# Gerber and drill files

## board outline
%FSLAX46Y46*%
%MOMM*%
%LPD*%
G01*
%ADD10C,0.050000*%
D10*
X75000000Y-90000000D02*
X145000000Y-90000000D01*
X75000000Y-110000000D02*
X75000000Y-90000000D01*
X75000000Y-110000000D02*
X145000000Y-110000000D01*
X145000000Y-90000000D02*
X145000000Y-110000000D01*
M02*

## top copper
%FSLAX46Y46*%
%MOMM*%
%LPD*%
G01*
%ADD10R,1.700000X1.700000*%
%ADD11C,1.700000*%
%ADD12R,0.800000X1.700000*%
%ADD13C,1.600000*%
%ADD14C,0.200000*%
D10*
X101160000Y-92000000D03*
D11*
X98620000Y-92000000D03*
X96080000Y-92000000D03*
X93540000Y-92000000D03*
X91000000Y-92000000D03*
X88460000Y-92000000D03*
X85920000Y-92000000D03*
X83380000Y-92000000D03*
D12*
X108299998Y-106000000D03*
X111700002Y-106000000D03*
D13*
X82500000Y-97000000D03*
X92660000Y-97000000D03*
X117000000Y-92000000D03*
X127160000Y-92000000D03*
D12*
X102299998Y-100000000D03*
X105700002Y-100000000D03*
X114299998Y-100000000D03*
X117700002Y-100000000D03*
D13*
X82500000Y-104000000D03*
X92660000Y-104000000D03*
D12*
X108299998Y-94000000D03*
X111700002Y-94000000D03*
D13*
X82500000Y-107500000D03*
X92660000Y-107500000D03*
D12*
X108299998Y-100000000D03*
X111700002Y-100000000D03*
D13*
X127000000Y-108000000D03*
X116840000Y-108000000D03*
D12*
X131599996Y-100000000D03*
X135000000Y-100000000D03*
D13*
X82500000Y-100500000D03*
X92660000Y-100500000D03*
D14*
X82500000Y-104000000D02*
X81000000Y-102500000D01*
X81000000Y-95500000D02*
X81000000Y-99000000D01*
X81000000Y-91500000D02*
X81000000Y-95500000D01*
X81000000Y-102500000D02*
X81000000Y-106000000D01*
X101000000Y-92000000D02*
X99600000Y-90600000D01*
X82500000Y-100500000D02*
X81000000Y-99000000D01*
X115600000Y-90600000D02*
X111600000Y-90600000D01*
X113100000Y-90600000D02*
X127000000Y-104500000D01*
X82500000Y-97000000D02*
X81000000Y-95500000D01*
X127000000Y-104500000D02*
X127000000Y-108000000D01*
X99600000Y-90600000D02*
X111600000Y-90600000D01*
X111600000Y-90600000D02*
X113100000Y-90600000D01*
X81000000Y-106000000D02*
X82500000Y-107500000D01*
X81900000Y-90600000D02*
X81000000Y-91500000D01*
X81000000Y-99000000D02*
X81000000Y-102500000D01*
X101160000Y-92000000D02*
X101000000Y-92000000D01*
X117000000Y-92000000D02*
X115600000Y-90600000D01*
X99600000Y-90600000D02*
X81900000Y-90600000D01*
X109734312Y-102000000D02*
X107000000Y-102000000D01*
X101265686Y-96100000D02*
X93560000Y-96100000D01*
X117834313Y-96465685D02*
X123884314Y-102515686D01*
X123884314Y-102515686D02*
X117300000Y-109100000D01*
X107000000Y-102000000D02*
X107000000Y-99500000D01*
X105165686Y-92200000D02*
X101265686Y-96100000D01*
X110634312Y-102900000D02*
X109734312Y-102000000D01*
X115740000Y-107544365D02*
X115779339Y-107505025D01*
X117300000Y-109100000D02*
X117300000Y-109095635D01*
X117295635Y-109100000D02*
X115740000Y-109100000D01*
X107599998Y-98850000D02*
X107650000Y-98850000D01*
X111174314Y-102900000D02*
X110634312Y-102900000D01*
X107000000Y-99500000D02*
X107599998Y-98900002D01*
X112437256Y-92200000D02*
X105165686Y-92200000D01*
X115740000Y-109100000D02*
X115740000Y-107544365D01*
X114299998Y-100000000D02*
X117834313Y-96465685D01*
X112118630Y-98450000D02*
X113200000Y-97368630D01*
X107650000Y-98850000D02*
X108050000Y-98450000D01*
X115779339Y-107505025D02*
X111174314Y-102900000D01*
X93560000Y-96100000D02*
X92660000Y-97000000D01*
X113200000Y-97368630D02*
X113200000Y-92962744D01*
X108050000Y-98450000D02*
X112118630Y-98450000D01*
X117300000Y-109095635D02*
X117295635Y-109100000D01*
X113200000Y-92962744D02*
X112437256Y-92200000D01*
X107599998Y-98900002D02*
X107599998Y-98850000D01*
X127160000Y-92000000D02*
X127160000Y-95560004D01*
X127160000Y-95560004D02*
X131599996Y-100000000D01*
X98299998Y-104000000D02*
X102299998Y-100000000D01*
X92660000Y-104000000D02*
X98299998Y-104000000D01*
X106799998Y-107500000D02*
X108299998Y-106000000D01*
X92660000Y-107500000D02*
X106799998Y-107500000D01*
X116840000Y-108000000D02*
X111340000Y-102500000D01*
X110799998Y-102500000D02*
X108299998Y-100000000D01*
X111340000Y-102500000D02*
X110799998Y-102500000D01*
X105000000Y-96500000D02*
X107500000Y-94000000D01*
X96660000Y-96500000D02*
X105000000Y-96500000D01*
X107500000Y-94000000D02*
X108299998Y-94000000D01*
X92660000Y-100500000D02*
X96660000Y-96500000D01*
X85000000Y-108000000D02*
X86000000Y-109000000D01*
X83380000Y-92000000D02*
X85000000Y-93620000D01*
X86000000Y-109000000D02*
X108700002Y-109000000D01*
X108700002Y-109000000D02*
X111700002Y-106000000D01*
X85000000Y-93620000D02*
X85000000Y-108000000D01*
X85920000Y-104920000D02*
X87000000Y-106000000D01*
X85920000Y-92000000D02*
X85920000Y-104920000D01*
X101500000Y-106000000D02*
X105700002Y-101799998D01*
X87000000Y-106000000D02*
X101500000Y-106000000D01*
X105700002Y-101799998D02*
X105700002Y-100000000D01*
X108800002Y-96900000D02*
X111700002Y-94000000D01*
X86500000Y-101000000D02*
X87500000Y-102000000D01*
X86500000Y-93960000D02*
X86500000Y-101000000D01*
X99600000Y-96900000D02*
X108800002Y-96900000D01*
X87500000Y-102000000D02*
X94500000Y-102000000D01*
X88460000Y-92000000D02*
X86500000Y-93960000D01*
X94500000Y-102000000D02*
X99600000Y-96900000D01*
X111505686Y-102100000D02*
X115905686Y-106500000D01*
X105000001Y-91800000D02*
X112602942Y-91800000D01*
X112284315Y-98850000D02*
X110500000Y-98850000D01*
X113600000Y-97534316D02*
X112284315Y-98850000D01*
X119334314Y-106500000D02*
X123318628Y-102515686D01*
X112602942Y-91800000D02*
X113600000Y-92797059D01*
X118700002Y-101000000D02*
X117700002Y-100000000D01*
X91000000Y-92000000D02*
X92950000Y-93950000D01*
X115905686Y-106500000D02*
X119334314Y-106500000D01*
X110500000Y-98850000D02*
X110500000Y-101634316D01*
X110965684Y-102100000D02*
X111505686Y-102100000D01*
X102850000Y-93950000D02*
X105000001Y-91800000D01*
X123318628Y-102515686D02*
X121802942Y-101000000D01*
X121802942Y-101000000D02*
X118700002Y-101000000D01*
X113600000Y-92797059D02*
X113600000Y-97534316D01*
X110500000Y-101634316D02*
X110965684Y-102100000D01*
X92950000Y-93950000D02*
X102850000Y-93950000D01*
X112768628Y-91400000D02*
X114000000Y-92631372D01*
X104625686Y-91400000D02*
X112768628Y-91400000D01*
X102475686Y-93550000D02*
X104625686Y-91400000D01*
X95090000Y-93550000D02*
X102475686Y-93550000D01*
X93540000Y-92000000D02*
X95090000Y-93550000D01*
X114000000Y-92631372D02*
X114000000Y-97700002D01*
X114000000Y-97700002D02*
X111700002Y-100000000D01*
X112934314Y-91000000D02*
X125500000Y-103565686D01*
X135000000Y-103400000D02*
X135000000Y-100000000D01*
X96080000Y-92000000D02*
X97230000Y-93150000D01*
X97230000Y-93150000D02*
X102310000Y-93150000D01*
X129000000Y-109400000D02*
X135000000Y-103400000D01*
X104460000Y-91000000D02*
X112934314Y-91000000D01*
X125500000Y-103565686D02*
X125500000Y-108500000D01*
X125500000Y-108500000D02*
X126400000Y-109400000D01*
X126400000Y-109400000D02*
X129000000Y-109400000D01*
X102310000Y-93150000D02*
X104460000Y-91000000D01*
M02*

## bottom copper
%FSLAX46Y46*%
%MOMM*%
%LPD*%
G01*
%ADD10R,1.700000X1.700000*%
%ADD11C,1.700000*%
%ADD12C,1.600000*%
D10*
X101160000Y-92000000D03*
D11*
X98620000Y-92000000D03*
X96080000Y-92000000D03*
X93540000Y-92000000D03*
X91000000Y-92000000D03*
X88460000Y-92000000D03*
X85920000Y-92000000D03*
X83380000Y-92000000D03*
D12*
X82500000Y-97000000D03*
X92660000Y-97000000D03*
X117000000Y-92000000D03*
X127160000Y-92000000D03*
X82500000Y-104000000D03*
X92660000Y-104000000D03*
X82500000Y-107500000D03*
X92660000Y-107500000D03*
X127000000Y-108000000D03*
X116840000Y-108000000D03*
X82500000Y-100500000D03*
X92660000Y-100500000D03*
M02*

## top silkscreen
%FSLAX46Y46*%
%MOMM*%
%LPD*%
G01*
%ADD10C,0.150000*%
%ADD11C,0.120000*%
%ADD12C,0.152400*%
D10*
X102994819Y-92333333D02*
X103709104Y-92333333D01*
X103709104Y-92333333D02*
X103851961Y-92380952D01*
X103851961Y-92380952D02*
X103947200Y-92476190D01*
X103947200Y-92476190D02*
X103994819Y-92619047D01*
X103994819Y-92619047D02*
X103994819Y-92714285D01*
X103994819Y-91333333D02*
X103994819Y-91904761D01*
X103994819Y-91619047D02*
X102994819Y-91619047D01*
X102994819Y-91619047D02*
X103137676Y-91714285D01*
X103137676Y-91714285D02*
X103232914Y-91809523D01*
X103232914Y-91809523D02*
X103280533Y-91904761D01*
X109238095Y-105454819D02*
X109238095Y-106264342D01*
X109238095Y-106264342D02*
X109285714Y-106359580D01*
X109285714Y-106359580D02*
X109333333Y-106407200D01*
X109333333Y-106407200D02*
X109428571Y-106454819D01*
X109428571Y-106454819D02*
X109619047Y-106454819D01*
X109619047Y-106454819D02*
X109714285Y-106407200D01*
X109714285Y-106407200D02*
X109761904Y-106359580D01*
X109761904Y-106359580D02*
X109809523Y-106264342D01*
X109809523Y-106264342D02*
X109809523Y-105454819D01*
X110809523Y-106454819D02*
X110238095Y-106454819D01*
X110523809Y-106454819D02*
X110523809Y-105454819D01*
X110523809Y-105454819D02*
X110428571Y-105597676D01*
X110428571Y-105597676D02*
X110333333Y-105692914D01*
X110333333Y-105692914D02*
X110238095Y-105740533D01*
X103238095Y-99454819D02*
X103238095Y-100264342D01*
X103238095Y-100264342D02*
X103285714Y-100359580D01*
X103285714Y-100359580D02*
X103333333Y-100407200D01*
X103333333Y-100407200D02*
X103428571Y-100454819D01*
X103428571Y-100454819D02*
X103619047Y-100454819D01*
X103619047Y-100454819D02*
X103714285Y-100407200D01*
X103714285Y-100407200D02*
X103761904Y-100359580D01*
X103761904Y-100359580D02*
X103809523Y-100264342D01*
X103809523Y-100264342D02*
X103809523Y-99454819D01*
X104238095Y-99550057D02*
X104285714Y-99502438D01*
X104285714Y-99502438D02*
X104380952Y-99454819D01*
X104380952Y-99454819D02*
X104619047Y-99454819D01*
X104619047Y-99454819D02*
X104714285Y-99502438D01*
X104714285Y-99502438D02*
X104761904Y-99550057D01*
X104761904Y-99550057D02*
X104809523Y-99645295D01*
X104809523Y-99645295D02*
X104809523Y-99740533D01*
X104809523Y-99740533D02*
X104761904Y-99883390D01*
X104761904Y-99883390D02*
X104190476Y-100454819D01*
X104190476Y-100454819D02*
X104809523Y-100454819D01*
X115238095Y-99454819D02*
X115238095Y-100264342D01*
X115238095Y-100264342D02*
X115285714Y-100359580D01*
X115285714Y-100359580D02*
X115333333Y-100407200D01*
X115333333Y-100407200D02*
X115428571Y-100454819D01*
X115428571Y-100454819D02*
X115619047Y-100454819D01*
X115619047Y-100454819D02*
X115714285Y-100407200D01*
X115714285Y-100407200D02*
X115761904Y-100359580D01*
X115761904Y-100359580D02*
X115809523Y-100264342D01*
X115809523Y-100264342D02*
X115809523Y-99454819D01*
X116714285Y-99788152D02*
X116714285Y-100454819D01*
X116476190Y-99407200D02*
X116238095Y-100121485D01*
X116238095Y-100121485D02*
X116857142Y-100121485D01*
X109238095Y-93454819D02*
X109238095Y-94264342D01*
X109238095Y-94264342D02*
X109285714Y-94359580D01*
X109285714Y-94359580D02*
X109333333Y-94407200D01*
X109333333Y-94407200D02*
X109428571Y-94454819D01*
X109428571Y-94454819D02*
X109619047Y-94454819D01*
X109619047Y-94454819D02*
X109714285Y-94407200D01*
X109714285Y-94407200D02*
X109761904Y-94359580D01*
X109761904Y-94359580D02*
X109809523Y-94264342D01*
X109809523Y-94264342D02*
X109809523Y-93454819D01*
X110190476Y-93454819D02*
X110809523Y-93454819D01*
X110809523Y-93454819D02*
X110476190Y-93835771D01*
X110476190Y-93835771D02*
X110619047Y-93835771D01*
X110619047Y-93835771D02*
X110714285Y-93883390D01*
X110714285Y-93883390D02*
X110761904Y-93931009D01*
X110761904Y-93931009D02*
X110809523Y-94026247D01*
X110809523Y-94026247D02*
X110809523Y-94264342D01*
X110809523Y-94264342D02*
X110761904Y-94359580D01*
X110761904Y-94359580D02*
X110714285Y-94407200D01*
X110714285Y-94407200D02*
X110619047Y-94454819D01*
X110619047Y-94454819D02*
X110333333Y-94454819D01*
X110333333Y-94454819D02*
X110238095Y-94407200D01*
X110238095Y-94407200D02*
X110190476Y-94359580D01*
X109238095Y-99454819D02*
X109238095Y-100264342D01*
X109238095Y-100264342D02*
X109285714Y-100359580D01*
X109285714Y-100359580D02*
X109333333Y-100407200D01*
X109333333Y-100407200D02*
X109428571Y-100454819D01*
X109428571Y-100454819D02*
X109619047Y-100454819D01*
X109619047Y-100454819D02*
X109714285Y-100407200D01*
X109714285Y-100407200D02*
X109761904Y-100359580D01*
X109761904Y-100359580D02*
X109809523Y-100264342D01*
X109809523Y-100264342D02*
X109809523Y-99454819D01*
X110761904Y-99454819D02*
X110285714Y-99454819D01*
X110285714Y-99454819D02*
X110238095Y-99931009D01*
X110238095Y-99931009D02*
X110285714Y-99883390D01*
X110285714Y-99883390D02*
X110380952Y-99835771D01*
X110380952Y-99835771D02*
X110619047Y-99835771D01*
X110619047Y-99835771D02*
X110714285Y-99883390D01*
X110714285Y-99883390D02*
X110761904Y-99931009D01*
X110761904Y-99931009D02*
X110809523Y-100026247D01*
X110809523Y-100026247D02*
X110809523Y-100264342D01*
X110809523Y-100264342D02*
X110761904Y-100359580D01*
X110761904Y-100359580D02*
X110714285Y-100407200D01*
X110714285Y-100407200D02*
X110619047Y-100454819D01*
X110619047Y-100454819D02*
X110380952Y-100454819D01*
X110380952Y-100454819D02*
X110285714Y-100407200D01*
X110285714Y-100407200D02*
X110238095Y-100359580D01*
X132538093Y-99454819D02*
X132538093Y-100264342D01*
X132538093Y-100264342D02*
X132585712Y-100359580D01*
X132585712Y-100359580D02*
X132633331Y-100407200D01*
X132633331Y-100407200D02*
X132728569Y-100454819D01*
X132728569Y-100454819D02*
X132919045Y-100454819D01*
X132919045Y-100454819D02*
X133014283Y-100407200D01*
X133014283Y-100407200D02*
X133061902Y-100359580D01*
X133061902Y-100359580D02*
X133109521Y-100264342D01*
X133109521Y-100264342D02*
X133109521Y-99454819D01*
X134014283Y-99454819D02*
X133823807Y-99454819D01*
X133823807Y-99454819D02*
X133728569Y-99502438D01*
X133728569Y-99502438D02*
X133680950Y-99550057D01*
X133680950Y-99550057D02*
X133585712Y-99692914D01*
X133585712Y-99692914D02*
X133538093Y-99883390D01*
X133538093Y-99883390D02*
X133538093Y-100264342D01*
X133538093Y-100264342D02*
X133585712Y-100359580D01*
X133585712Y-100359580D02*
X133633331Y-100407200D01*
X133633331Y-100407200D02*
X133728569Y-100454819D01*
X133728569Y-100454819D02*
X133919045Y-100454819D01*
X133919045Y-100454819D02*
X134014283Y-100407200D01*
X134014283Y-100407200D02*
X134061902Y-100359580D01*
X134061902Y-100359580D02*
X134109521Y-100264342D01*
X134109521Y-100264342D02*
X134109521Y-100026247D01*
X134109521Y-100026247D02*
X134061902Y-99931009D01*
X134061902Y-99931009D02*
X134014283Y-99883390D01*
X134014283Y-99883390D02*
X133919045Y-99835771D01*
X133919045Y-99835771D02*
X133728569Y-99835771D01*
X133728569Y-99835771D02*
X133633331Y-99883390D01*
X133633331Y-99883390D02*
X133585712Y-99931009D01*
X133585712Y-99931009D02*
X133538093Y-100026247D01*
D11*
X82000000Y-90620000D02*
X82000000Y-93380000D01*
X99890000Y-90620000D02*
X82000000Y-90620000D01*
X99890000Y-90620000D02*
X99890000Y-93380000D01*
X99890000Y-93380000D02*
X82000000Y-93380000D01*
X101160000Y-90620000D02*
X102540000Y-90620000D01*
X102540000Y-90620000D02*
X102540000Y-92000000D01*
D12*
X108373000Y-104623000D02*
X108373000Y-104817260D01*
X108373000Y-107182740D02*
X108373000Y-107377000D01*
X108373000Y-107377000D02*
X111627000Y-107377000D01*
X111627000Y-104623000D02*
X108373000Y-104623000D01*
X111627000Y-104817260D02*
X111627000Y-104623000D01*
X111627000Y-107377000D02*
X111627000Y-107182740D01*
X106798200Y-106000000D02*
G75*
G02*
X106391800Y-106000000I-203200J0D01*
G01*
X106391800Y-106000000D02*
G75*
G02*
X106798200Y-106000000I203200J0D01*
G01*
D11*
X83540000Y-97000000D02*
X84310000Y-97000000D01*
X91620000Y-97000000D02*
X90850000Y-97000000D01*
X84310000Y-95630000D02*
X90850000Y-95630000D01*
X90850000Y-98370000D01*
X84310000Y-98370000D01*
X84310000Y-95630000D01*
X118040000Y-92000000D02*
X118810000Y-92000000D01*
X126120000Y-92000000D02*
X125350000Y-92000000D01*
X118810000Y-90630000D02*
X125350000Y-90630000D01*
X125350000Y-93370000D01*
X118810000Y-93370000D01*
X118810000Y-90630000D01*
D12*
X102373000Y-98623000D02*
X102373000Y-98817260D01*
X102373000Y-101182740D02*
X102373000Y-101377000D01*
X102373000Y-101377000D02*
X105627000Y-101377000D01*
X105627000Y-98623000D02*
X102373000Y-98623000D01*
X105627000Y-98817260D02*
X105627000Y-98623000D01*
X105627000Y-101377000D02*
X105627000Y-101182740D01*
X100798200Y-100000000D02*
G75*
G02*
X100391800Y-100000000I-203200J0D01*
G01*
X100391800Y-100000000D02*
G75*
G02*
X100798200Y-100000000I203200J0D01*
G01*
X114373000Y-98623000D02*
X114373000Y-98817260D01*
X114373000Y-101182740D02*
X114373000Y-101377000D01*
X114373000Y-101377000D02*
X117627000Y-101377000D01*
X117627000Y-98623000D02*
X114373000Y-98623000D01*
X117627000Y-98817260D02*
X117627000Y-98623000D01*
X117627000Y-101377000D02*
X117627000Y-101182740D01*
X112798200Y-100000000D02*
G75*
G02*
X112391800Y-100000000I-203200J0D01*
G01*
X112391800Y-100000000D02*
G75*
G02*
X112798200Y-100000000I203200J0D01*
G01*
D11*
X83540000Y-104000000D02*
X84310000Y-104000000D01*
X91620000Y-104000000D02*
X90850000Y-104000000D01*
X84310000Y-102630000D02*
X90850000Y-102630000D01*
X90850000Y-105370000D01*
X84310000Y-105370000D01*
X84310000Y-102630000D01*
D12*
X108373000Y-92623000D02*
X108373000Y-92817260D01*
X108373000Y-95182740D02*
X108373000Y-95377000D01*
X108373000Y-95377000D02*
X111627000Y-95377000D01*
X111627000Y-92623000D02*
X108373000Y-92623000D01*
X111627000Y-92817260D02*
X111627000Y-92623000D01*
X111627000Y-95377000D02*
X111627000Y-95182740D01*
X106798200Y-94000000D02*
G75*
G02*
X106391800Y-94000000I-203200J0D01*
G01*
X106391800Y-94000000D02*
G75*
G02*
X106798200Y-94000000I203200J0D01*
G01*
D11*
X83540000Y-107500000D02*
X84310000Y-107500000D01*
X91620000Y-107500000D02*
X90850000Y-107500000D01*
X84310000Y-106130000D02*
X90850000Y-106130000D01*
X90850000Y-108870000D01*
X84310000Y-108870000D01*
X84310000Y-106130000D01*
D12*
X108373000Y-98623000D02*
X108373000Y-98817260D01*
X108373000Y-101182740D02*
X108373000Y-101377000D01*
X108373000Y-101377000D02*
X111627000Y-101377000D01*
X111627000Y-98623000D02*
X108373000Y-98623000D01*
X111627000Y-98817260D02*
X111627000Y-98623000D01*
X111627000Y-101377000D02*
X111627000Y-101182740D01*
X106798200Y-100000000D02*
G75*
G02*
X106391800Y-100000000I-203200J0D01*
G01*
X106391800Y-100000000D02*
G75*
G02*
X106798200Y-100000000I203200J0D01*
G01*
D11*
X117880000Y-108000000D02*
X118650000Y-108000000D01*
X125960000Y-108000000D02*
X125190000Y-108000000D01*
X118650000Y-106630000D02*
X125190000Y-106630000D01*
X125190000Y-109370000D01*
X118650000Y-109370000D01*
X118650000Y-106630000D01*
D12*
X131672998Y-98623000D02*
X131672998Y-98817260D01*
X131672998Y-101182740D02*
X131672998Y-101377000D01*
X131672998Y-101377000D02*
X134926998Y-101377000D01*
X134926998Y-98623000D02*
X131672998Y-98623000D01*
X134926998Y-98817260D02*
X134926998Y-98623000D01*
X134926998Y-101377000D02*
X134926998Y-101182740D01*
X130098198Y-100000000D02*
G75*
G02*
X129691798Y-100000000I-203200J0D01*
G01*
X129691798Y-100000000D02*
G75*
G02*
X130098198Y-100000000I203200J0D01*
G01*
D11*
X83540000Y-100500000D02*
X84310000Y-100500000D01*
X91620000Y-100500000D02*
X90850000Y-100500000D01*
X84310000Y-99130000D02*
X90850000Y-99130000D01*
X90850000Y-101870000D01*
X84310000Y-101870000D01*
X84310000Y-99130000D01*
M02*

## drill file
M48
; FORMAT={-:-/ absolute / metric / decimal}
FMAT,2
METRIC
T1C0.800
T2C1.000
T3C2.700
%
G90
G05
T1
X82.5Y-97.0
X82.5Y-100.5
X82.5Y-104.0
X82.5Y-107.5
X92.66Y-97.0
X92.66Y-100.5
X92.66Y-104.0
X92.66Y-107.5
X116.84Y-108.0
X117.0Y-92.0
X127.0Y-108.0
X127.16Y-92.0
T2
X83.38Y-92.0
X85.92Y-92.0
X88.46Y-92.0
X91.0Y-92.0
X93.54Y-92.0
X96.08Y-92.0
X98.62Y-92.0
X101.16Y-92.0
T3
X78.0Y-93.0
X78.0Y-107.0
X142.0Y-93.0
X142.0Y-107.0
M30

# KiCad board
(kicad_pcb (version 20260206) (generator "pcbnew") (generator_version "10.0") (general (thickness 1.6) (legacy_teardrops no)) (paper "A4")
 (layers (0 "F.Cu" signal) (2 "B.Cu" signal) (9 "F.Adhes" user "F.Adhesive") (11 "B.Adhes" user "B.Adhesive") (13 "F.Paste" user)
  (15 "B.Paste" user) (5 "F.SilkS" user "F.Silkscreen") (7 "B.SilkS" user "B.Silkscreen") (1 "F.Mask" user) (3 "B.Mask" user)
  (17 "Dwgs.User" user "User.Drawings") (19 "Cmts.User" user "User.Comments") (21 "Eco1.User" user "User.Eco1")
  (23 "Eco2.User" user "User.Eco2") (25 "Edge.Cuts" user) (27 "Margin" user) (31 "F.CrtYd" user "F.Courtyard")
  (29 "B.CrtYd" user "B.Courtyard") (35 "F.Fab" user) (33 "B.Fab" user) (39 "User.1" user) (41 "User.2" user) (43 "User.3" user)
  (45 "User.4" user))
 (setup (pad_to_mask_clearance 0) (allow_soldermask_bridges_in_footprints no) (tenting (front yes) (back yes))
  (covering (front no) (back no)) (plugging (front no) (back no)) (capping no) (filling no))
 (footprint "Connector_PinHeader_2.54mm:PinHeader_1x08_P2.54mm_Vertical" (layer "F.Cu") (at 101.16 92 -90)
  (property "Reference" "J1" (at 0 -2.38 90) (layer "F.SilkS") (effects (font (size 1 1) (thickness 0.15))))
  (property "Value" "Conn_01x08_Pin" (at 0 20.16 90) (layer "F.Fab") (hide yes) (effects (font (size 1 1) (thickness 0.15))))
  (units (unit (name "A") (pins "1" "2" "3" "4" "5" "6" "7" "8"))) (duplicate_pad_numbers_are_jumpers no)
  (fp_line (start -1.38 19.16) (end 1.38 19.16) (stroke (width 0.12) (type solid)) (layer "F.SilkS"))
  (fp_line (start -1.38 1.27) (end -1.38 19.16) (stroke (width 0.12) (type solid)) (layer "F.SilkS"))
  (fp_line (start -1.38 1.27) (end 1.38 1.27) (stroke (width 0.12) (type solid)) (layer "F.SilkS"))
  (fp_line (start 1.38 1.27) (end 1.38 19.16) (stroke (width 0.12) (type solid)) (layer "F.SilkS"))
  (fp_line (start -1.38 0) (end -1.38 -1.38) (stroke (width 0.12) (type solid)) (layer "F.SilkS"))
  (fp_line (start -1.38 -1.38) (end 0 -1.38) (stroke (width 0.12) (type solid)) (layer "F.SilkS"))
  (pad "1" thru_hole rect (at 0 0 270) (size 1.7 1.7) (drill 1) (layers "*.Cu" "*.Mask") (remove_unused_layers no) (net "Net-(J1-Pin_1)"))
  (pad "2" thru_hole circle (at 0 2.54 270) (size 1.7 1.7) (drill 1) (layers "*.Cu" "*.Mask") (remove_unused_layers no)
   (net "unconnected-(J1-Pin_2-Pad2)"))
  (pad "3" thru_hole circle (at 0 5.08 270) (size 1.7 1.7) (drill 1) (layers "*.Cu" "*.Mask") (remove_unused_layers no) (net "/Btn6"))
  (pad "4" thru_hole circle (at 0 7.62 270) (size 1.7 1.7) (drill 1) (layers "*.Cu" "*.Mask") (remove_unused_layers no) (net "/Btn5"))
  (pad "5" thru_hole circle (at 0 10.16 270) (size 1.7 1.7) (drill 1) (layers "*.Cu" "*.Mask") (remove_unused_layers no) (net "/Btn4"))
  (pad "6" thru_hole circle (at 0 12.7 270) (size 1.7 1.7) (drill 1) (layers "*.Cu" "*.Mask") (remove_unused_layers no) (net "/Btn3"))
  (pad "7" thru_hole circle (at 0 15.24 270) (size 1.7 1.7) (drill 1) (layers "*.Cu" "*.Mask") (remove_unused_layers no) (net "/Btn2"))
  (pad "8" thru_hole circle (at 0 17.78 270) (size 1.7 1.7) (drill 1) (layers "*.Cu" "*.Mask") (remove_unused_layers no) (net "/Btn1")))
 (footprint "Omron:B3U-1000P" (layer "F.Cu") (at 110 106)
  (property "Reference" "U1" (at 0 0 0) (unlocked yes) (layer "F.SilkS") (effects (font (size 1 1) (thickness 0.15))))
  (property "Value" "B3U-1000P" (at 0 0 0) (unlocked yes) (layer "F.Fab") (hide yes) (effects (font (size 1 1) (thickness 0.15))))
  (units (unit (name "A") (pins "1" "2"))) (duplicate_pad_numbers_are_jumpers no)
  (fp_line (start -1.627 -1.377) (end -1.627 -1.18274) (stroke (width 0.1524) (type solid)) (layer "F.SilkS"))
  (fp_line (start -1.627 1.18274) (end -1.627 1.377) (stroke (width 0.1524) (type solid)) (layer "F.SilkS"))
  (fp_line (start -1.627 1.377) (end 1.627 1.377) (stroke (width 0.1524) (type solid)) (layer "F.SilkS"))
  (fp_line (start 1.627 -1.377) (end -1.627 -1.377) (stroke (width 0.1524) (type solid)) (layer "F.SilkS"))
  (fp_line (start 1.627 -1.18274) (end 1.627 -1.377) (stroke (width 0.1524) (type solid)) (layer "F.SilkS"))
  (fp_line (start 1.627 1.377) (end 1.627 1.18274) (stroke (width 0.1524) (type solid)) (layer "F.SilkS"))
  (fp_circle (center -3.405 0) (end -3.2018 0) (stroke (width 0.1524) (type solid)) (fill no) (layer "F.SilkS"))
  (pad "1" smd rect (at -1.700002 0) (size 0.8 1.7) (layers "F.Cu" "F.Mask" "F.Paste") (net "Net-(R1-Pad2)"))
  (pad "2" smd rect (at 1.700002 0) (size 0.8 1.7) (layers "F.Cu" "F.Mask" "F.Paste") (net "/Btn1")))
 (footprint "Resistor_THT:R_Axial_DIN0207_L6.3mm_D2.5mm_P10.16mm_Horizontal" (layer "F.Cu") (at 82.5 97)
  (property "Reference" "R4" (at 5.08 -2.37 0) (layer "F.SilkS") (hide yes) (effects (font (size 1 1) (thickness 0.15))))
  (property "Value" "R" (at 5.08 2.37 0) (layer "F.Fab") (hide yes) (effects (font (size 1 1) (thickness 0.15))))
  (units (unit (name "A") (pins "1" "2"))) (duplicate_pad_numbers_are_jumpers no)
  (fp_line (start 1.04 0) (end 1.81 0) (stroke (width 0.12) (type solid)) (layer "F.SilkS"))
  (fp_line (start 9.12 0) (end 8.35 0) (stroke (width 0.12) (type solid)) (layer "F.SilkS"))
  (fp_rect (start 1.81 -1.37) (end 8.35 1.37) (stroke (width 0.12) (type solid)) (fill no) (layer "F.SilkS"))
  (pad "1" thru_hole circle (at 0 0) (size 1.6 1.6) (drill 0.8) (layers "*.Cu" "*.Mask") (remove_unused_layers no) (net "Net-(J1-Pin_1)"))
  (pad "2" thru_hole circle (at 10.16 0) (size 1.6 1.6) (drill 0.8) (layers "*.Cu" "*.Mask") (remove_unused_layers no) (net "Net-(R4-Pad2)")))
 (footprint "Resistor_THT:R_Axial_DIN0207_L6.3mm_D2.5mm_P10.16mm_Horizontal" (layer "F.Cu") (at 117 92)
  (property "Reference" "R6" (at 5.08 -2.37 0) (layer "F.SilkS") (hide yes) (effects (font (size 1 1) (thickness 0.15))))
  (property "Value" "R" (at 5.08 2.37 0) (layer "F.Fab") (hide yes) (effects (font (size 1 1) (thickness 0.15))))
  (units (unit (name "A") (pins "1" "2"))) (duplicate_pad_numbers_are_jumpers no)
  (fp_line (start 1.04 0) (end 1.81 0) (stroke (width 0.12) (type solid)) (layer "F.SilkS"))
  (fp_line (start 9.12 0) (end 8.35 0) (stroke (width 0.12) (type solid)) (layer "F.SilkS"))
  (fp_rect (start 1.81 -1.37) (end 8.35 1.37) (stroke (width 0.12) (type solid)) (fill no) (layer "F.SilkS"))
  (pad "1" thru_hole circle (at 0 0) (size 1.6 1.6) (drill 0.8) (layers "*.Cu" "*.Mask") (remove_unused_layers no) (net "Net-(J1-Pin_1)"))
  (pad "2" thru_hole circle (at 10.16 0) (size 1.6 1.6) (drill 0.8) (layers "*.Cu" "*.Mask") (remove_unused_layers no) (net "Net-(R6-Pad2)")))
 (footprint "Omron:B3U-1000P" (layer "F.Cu") (at 104 100)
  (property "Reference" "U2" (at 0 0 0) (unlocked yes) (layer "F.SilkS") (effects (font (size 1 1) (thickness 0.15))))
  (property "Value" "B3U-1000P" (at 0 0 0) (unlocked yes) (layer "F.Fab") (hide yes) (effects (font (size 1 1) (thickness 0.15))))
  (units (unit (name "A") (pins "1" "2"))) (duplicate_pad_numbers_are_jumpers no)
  (fp_line (start -1.627 -1.377) (end -1.627 -1.18274) (stroke (width 0.1524) (type solid)) (layer "F.SilkS"))
  (fp_line (start -1.627 1.18274) (end -1.627 1.377) (stroke (width 0.1524) (type solid)) (layer "F.SilkS"))
  (fp_line (start -1.627 1.377) (end 1.627 1.377) (stroke (width 0.1524) (type solid)) (layer "F.SilkS"))
  (fp_line (start 1.627 -1.377) (end -1.627 -1.377) (stroke (width 0.1524) (type solid)) (layer "F.SilkS"))
  (fp_line (start 1.627 -1.18274) (end 1.627 -1.377) (stroke (width 0.1524) (type solid)) (layer "F.SilkS"))
  (fp_line (start 1.627 1.377) (end 1.627 1.18274) (stroke (width 0.1524) (type solid)) (layer "F.SilkS"))
  (fp_circle (center -3.405 0) (end -3.2018 0) (stroke (width 0.1524) (type solid)) (fill no) (layer "F.SilkS"))
  (pad "1" smd rect (at -1.700002 0) (size 0.8 1.7) (layers "F.Cu" "F.Mask" "F.Paste") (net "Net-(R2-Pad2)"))
  (pad "2" smd rect (at 1.700002 0) (size 0.8 1.7) (layers "F.Cu" "F.Mask" "F.Paste") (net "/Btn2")))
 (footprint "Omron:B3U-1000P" (layer "F.Cu") (at 116 100)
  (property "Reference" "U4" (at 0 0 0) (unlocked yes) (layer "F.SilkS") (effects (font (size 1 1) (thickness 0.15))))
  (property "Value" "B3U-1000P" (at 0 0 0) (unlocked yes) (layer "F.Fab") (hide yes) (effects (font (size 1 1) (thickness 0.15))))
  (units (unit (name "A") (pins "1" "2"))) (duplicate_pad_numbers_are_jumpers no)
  (fp_line (start -1.627 -1.377) (end -1.627 -1.18274) (stroke (width 0.1524) (type solid)) (layer "F.SilkS"))
  (fp_line (start -1.627 1.18274) (end -1.627 1.377) (stroke (width 0.1524) (type solid)) (layer "F.SilkS"))
  (fp_line (start -1.627 1.377) (end 1.627 1.377) (stroke (width 0.1524) (type solid)) (layer "F.SilkS"))
  (fp_line (start 1.627 -1.377) (end -1.627 -1.377) (stroke (width 0.1524) (type solid)) (layer "F.SilkS"))
  (fp_line (start 1.627 -1.18274) (end 1.627 -1.377) (stroke (width 0.1524) (type solid)) (layer "F.SilkS"))
  (fp_line (start 1.627 1.377) (end 1.627 1.18274) (stroke (width 0.1524) (type solid)) (layer "F.SilkS"))
  (fp_circle (center -3.405 0) (end -3.2018 0) (stroke (width 0.1524) (type solid)) (fill no) (layer "F.SilkS"))
  (pad "1" smd rect (at -1.700002 0) (size 0.8 1.7) (layers "F.Cu" "F.Mask" "F.Paste") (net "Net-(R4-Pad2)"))
  (pad "2" smd rect (at 1.700002 0) (size 0.8 1.7) (layers "F.Cu" "F.Mask" "F.Paste") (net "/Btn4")))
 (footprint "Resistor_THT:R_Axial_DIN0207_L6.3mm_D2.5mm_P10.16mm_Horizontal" (layer "F.Cu") (at 82.5 104)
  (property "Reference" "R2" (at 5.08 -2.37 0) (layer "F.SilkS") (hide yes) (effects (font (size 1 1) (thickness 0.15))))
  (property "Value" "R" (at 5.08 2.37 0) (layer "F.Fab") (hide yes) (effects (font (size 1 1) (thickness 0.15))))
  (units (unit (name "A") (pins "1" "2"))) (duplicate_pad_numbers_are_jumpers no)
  (fp_line (start 1.04 0) (end 1.81 0) (stroke (width 0.12) (type solid)) (layer "F.SilkS"))
  (fp_line (start 9.12 0) (end 8.35 0) (stroke (width 0.12) (type solid)) (layer "F.SilkS"))
  (fp_rect (start 1.81 -1.37) (end 8.35 1.37) (stroke (width 0.12) (type solid)) (fill no) (layer "F.SilkS"))
  (pad "1" thru_hole circle (at 0 0) (size 1.6 1.6) (drill 0.8) (layers "*.Cu" "*.Mask") (remove_unused_layers no) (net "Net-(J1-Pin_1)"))
  (pad "2" thru_hole circle (at 10.16 0) (size 1.6 1.6) (drill 0.8) (layers "*.Cu" "*.Mask") (remove_unused_layers no) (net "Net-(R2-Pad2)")))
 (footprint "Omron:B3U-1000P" (layer "F.Cu") (at 110 94)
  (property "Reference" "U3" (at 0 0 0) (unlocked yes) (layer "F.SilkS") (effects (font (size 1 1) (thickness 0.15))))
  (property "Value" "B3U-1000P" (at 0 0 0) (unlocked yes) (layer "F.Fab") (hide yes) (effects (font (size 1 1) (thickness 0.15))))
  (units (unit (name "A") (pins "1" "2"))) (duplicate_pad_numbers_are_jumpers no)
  (fp_line (start -1.627 -1.377) (end -1.627 -1.18274) (stroke (width 0.1524) (type solid)) (layer "F.SilkS"))
  (fp_line (start -1.627 1.18274) (end -1.627 1.377) (stroke (width 0.1524) (type solid)) (layer "F.SilkS"))
  (fp_line (start -1.627 1.377) (end 1.627 1.377) (stroke (width 0.1524) (type solid)) (layer "F.SilkS"))
  (fp_line (start 1.627 -1.377) (end -1.627 -1.377) (stroke (width 0.1524) (type solid)) (layer "F.SilkS"))
  (fp_line (start 1.627 -1.18274) (end 1.627 -1.377) (stroke (width 0.1524) (type solid)) (layer "F.SilkS"))
  (fp_line (start 1.627 1.377) (end 1.627 1.18274) (stroke (width 0.1524) (type solid)) (layer "F.SilkS"))
  (fp_circle (center -3.405 0) (end -3.2018 0) (stroke (width 0.1524) (type solid)) (fill no) (layer "F.SilkS"))
  (pad "1" smd rect (at -1.700002 0) (size 0.8 1.7) (layers "F.Cu" "F.Mask" "F.Paste") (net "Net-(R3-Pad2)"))
  (pad "2" smd rect (at 1.700002 0) (size 0.8 1.7) (layers "F.Cu" "F.Mask" "F.Paste") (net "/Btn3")))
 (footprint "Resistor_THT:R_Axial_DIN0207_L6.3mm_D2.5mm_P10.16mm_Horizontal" (layer "F.Cu") (at 82.5 107.5)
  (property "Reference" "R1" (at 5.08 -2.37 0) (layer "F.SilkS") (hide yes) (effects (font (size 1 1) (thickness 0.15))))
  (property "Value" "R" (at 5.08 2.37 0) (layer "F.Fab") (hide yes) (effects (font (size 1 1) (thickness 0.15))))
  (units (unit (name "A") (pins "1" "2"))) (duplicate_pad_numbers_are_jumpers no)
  (fp_line (start 1.04 0) (end 1.81 0) (stroke (width 0.12) (type solid)) (layer "F.SilkS"))
  (fp_line (start 9.12 0) (end 8.35 0) (stroke (width 0.12) (type solid)) (layer "F.SilkS"))
  (fp_rect (start 1.81 -1.37) (end 8.35 1.37) (stroke (width 0.12) (type solid)) (fill no) (layer "F.SilkS"))
  (pad "1" thru_hole circle (at 0 0) (size 1.6 1.6) (drill 0.8) (layers "*.Cu" "*.Mask") (remove_unused_layers no) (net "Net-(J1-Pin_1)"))
  (pad "2" thru_hole circle (at 10.16 0) (size 1.6 1.6) (drill 0.8) (layers "*.Cu" "*.Mask") (remove_unused_layers no) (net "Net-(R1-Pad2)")))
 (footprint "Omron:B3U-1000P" (layer "F.Cu") (at 110 100)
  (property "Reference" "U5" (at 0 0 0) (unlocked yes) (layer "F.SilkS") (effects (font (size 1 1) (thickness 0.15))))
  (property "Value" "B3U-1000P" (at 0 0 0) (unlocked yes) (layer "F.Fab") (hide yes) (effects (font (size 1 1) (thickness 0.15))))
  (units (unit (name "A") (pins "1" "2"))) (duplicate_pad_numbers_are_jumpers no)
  (fp_line (start -1.627 -1.377) (end -1.627 -1.18274) (stroke (width 0.1524) (type solid)) (layer "F.SilkS"))
  (fp_line (start -1.627 1.18274) (end -1.627 1.377) (stroke (width 0.1524) (type solid)) (layer "F.SilkS"))
  (fp_line (start -1.627 1.377) (end 1.627 1.377) (stroke (width 0.1524) (type solid)) (layer "F.SilkS"))
  (fp_line (start 1.627 -1.377) (end -1.627 -1.377) (stroke (width 0.1524) (type solid)) (layer "F.SilkS"))
  (fp_line (start 1.627 -1.18274) (end 1.627 -1.377) (stroke (width 0.1524) (type solid)) (layer "F.SilkS"))
  (fp_line (start 1.627 1.377) (end 1.627 1.18274) (stroke (width 0.1524) (type solid)) (layer "F.SilkS"))
  (fp_circle (center -3.405 0) (end -3.2018 0) (stroke (width 0.1524) (type solid)) (fill no) (layer "F.SilkS"))
  (pad "1" smd rect (at -1.700002 0) (size 0.8 1.7) (layers "F.Cu" "F.Mask" "F.Paste") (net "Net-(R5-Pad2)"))
  (pad "2" smd rect (at 1.700002 0) (size 0.8 1.7) (layers "F.Cu" "F.Mask" "F.Paste") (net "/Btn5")))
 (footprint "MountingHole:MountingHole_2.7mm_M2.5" (layer "F.Cu") (at 142 93)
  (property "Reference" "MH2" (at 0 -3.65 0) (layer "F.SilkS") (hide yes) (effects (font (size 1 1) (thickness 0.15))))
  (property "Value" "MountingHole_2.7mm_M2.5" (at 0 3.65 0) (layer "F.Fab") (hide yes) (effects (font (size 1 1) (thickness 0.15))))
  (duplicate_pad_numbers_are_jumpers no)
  (pad "" np_thru_hole circle (at 0 0) (size 2.7 2.7) (drill 2.7) (layers "*.Cu" "*.Mask")))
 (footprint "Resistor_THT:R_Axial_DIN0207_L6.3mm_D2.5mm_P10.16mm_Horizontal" (layer "F.Cu") (at 127 108 180)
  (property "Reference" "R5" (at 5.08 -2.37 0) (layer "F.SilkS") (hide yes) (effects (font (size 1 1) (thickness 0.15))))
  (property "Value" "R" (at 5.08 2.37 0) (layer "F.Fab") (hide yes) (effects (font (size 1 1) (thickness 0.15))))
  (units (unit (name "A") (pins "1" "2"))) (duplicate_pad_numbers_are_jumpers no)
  (fp_line (start 9.12 0) (end 8.35 0) (stroke (width 0.12) (type solid)) (layer "F.SilkS"))
  (fp_line (start 1.04 0) (end 1.81 0) (stroke (width 0.12) (type solid)) (layer "F.SilkS"))
  (fp_rect (start 1.81 -1.37) (end 8.35 1.37) (stroke (width 0.12) (type solid)) (fill no) (layer "F.SilkS"))
  (pad "1" thru_hole circle (at 0 0 180) (size 1.6 1.6) (drill 0.8) (layers "*.Cu" "*.Mask") (remove_unused_layers no)
   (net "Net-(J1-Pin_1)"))
  (pad "2" thru_hole circle (at 10.16 0 180) (size 1.6 1.6) (drill 0.8) (layers "*.Cu" "*.Mask") (remove_unused_layers no)
   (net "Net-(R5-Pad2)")))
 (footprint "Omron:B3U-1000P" (layer "F.Cu") (at 133.299998 100)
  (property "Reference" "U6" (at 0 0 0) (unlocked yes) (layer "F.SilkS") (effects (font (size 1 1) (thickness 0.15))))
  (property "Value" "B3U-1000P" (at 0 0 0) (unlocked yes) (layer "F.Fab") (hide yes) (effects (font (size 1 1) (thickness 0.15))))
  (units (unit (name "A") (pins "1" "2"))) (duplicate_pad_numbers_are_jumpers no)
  (fp_line (start -1.627 -1.377) (end -1.627 -1.18274) (stroke (width 0.1524) (type solid)) (layer "F.SilkS"))
  (fp_line (start -1.627 1.18274) (end -1.627 1.377) (stroke (width 0.1524) (type solid)) (layer "F.SilkS"))
  (fp_line (start -1.627 1.377) (end 1.627 1.377) (stroke (width 0.1524) (type solid)) (layer "F.SilkS"))
  (fp_line (start 1.627 -1.377) (end -1.627 -1.377) (stroke (width 0.1524) (type solid)) (layer "F.SilkS"))
  (fp_line (start 1.627 -1.18274) (end 1.627 -1.377) (stroke (width 0.1524) (type solid)) (layer "F.SilkS"))
  (fp_line (start 1.627 1.377) (end 1.627 1.18274) (stroke (width 0.1524) (type solid)) (layer "F.SilkS"))
  (fp_circle (center -3.405 0) (end -3.2018 0) (stroke (width 0.1524) (type solid)) (fill no) (layer "F.SilkS"))
  (pad "1" smd rect (at -1.700002 0) (size 0.8 1.7) (layers "F.Cu" "F.Mask" "F.Paste") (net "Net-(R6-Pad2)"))
  (pad "2" smd rect (at 1.700002 0) (size 0.8 1.7) (layers "F.Cu" "F.Mask" "F.Paste") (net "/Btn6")))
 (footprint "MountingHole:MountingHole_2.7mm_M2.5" (layer "F.Cu") (at 78 93)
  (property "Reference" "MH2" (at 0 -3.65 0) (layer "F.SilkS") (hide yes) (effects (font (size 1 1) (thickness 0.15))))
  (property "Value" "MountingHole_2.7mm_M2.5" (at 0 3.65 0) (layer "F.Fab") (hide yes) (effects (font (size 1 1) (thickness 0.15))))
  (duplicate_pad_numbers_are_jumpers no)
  (pad "" np_thru_hole circle (at 0 0) (size 2.7 2.7) (drill 2.7) (layers "*.Cu" "*.Mask")))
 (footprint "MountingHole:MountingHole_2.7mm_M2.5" (layer "F.Cu") (at 78 107)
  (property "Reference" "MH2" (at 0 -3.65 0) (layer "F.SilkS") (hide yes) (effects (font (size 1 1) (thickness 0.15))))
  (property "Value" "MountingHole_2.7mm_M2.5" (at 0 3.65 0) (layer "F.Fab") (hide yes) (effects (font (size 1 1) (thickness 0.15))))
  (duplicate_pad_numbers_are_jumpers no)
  (pad "" np_thru_hole circle (at 0 0) (size 2.7 2.7) (drill 2.7) (layers "*.Cu" "*.Mask")))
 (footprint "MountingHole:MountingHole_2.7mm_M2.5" (layer "F.Cu") (at 142 107)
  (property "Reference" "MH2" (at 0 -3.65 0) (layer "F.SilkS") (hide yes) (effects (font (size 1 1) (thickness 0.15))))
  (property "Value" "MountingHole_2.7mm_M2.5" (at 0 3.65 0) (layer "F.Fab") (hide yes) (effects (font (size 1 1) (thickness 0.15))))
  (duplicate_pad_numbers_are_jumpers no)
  (pad "" np_thru_hole circle (at 0 0) (size 2.7 2.7) (drill 2.7) (layers "*.Cu" "*.Mask")))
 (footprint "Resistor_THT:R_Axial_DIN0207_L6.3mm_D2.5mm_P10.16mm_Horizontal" (layer "F.Cu") (at 82.5 100.5)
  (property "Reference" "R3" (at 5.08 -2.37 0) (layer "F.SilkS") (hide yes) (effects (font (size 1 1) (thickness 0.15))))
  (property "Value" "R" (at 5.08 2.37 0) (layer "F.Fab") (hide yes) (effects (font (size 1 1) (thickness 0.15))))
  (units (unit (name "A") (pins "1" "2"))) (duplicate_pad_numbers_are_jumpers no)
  (fp_line (start 1.04 0) (end 1.81 0) (stroke (width 0.12) (type solid)) (layer "F.SilkS"))
  (fp_line (start 9.12 0) (end 8.35 0) (stroke (width 0.12) (type solid)) (layer "F.SilkS"))
  (fp_rect (start 1.81 -1.37) (end 8.35 1.37) (stroke (width 0.12) (type solid)) (fill no) (layer "F.SilkS"))
  (pad "1" thru_hole circle (at 0 0) (size 1.6 1.6) (drill 0.8) (layers "*.Cu" "*.Mask") (remove_unused_layers no) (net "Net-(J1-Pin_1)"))
  (pad "2" thru_hole circle (at 10.16 0) (size 1.6 1.6) (drill 0.8) (layers "*.Cu" "*.Mask") (remove_unused_layers no) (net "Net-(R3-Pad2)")))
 (gr_line (start 75 90) (end 145 90) (stroke (width 0.05) (type default)) (layer "Edge.Cuts"))
 (gr_line (start 75 110) (end 75 90) (stroke (width 0.05) (type default)) (layer "Edge.Cuts"))
 (gr_line (start 75 110) (end 145 110) (stroke (width 0.05) (type default)) (layer "Edge.Cuts"))
 (gr_line (start 145 90) (end 145 110) (stroke (width 0.05) (type default)) (layer "Edge.Cuts"))
 (segment (start 82.5 104) (end 81 102.5) (width 0.2) (layer "F.Cu") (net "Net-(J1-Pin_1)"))
 (segment (start 81 95.5) (end 81 99) (width 0.2) (layer "F.Cu") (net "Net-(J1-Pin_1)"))
 (segment (start 81 91.5) (end 81 95.5) (width 0.2) (layer "F.Cu") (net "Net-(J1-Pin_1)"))
 (segment (start 81 102.5) (end 81 106) (width 0.2) (layer "F.Cu") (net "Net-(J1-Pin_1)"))
 (segment (start 101 92) (end 99.6 90.6) (width 0.2) (layer "F.Cu") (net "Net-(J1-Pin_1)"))
 (segment (start 82.5 100.5) (end 81 99) (width 0.2) (layer "F.Cu") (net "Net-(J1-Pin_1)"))
 (segment (start 115.6 90.6) (end 111.6 90.6) (width 0.2) (layer "F.Cu") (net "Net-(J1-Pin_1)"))
 (segment (start 113.1 90.6) (end 127 104.5) (width 0.2) (layer "F.Cu") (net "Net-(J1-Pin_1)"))
 (segment (start 82.5 97) (end 81 95.5) (width 0.2) (layer "F.Cu") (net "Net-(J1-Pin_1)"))
 (segment (start 127 104.5) (end 127 108) (width 0.2) (layer "F.Cu") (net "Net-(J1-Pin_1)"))
 (segment (start 99.6 90.6) (end 111.6 90.6) (width 0.2) (layer "F.Cu") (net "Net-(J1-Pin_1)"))
 (segment (start 111.6 90.6) (end 113.1 90.6) (width 0.2) (layer "F.Cu") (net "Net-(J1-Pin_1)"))
 (segment (start 81 106) (end 82.5 107.5) (width 0.2) (layer "F.Cu") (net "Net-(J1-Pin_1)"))
 (segment (start 81.9 90.6) (end 81 91.5) (width 0.2) (layer "F.Cu") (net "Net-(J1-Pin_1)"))
 (segment (start 81 99) (end 81 102.5) (width 0.2) (layer "F.Cu") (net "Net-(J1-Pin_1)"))
 (segment (start 101.16 92) (end 101 92) (width 0.2) (layer "F.Cu") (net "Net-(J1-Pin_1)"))
 (segment (start 117 92) (end 115.6 90.6) (width 0.2) (layer "F.Cu") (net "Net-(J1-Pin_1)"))
 (segment (start 99.6 90.6) (end 81.9 90.6) (width 0.2) (layer "F.Cu") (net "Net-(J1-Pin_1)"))
 (segment (start 109.734312 102) (end 107 102) (width 0.2) (layer "F.Cu") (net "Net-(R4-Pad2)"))
 (segment (start 101.265686 96.1) (end 93.56 96.1) (width 0.2) (layer "F.Cu") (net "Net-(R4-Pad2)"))
 (segment (start 117.834313 96.465685) (end 123.884314 102.515686) (width 0.2) (layer "F.Cu") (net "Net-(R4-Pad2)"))
 (segment (start 123.884314 102.515686) (end 117.3 109.1) (width 0.2) (layer "F.Cu") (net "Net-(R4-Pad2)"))
 (segment (start 107 102) (end 107 99.5) (width 0.2) (layer "F.Cu") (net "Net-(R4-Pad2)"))
 (segment (start 105.165686 92.2) (end 101.265686 96.1) (width 0.2) (layer "F.Cu") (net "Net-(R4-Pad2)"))
 (segment (start 110.634312 102.9) (end 109.734312 102) (width 0.2) (layer "F.Cu") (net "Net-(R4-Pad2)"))
 (segment (start 115.74 107.544365) (end 115.779339 107.505025) (width 0.2) (layer "F.Cu") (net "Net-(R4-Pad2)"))
 (segment (start 117.3 109.1) (end 117.3 109.095635) (width 0.2) (layer "F.Cu") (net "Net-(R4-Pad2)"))
 (segment (start 117.295635 109.1) (end 115.74 109.1) (width 0.2) (layer "F.Cu") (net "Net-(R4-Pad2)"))
 (segment (start 107.599998 98.85) (end 107.65 98.85) (width 0.2) (layer "F.Cu") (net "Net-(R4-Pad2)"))
 (segment (start 111.174314 102.9) (end 110.634312 102.9) (width 0.2) (layer "F.Cu") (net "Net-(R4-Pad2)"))
 (segment (start 107 99.5) (end 107.599998 98.900002) (width 0.2) (layer "F.Cu") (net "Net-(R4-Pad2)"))
 (segment (start 112.437256 92.2) (end 105.165686 92.2) (width 0.2) (layer "F.Cu") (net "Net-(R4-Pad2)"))
 (segment (start 115.74 109.1) (end 115.74 107.544365) (width 0.2) (layer "F.Cu") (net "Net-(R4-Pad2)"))
 (segment (start 114.299998 100) (end 117.834313 96.465685) (width 0.2) (layer "F.Cu") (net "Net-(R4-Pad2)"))
 (segment (start 112.11863 98.45) (end 113.2 97.36863) (width 0.2) (layer "F.Cu") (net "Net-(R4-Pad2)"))
 (segment (start 107.65 98.85) (end 108.05 98.45) (width 0.2) (layer "F.Cu") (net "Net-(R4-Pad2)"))
 (segment (start 115.779339 107.505025) (end 111.174314 102.9) (width 0.2) (layer "F.Cu") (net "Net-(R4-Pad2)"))
 (segment (start 93.56 96.1) (end 92.66 97) (width 0.2) (layer "F.Cu") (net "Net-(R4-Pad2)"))
 (segment (start 113.2 97.36863) (end 113.2 92.962744) (width 0.2) (layer "F.Cu") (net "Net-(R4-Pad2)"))
 (segment (start 108.05 98.45) (end 112.11863 98.45) (width 0.2) (layer "F.Cu") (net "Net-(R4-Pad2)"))
 (segment (start 117.3 109.095635) (end 117.295635 109.1) (width 0.2) (layer "F.Cu") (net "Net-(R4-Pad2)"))
 (segment (start 113.2 92.962744) (end 112.437256 92.2) (width 0.2) (layer "F.Cu") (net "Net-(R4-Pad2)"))
 (segment (start 107.599998 98.900002) (end 107.599998 98.85) (width 0.2) (layer "F.Cu") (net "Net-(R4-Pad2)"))
 (segment (start 127.16 92) (end 127.16 95.560004) (width 0.2) (layer "F.Cu") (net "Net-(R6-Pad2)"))
 (segment (start 127.16 95.560004) (end 131.599996 100) (width 0.2) (layer "F.Cu") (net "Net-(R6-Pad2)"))
 (segment (start 98.299998 104) (end 102.299998 100) (width 0.2) (layer "F.Cu") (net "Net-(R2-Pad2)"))
 (segment (start 92.66 104) (end 98.299998 104) (width 0.2) (layer "F.Cu") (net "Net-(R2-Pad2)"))
 (segment (start 106.799998 107.5) (end 108.299998 106) (width 0.2) (layer "F.Cu") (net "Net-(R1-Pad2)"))
 (segment (start 92.66 107.5) (end 106.799998 107.5) (width 0.2) (layer "F.Cu") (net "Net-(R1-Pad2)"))
 (segment (start 116.84 108) (end 111.34 102.5) (width 0.2) (layer "F.Cu") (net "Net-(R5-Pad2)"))
 (segment (start 110.799998 102.5) (end 108.299998 100) (width 0.2) (layer "F.Cu") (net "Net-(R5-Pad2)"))
 (segment (start 111.34 102.5) (end 110.799998 102.5) (width 0.2) (layer "F.Cu") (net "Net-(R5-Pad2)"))
 (segment (start 105 96.5) (end 107.5 94) (width 0.2) (layer "F.Cu") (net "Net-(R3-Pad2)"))
 (segment (start 96.66 96.5) (end 105 96.5) (width 0.2) (layer "F.Cu") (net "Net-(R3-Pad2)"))
 (segment (start 107.5 94) (end 108.299998 94) (width 0.2) (layer "F.Cu") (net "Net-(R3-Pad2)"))
 (segment (start 92.66 100.5) (end 96.66 96.5) (width 0.2) (layer "F.Cu") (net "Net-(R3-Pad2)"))
 (segment (start 85 108) (end 86 109) (width 0.2) (layer "F.Cu") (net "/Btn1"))
 (segment (start 83.38 92) (end 85 93.62) (width 0.2) (layer "F.Cu") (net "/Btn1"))
 (segment (start 86 109) (end 108.700002 109) (width 0.2) (layer "F.Cu") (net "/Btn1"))
 (segment (start 108.700002 109) (end 111.700002 106) (width 0.2) (layer "F.Cu") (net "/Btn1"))
 (segment (start 85 93.62) (end 85 108) (width 0.2) (layer "F.Cu") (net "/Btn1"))
 (segment (start 85.92 104.92) (end 87 106) (width 0.2) (layer "F.Cu") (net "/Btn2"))
 (segment (start 85.92 92) (end 85.92 104.92) (width 0.2) (layer "F.Cu") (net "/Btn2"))
 (segment (start 101.5 106) (end 105.700002 101.799998) (width 0.2) (layer "F.Cu") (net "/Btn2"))
 (segment (start 87 106) (end 101.5 106) (width 0.2) (layer "F.Cu") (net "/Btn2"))
 (segment (start 105.700002 101.799998) (end 105.700002 100) (width 0.2) (layer "F.Cu") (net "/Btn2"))
 (segment (start 108.800002 96.9) (end 111.700002 94) (width 0.2) (layer "F.Cu") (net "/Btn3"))
 (segment (start 86.5 101) (end 87.5 102) (width 0.2) (layer "F.Cu") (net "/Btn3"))
 (segment (start 86.5 93.96) (end 86.5 101) (width 0.2) (layer "F.Cu") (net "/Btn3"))
 (segment (start 99.6 96.9) (end 108.800002 96.9) (width 0.2) (layer "F.Cu") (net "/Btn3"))
 (segment (start 87.5 102) (end 94.5 102) (width 0.2) (layer "F.Cu") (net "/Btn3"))
 (segment (start 88.46 92) (end 86.5 93.96) (width 0.2) (layer "F.Cu") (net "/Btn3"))
 (segment (start 94.5 102) (end 99.6 96.9) (width 0.2) (layer "F.Cu") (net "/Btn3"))
 (segment (start 111.505686 102.1) (end 115.905686 106.5) (width 0.2) (layer "F.Cu") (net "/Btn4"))
 (segment (start 105.000001 91.8) (end 112.602942 91.8) (width 0.2) (layer "F.Cu") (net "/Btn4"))
 (segment (start 112.284315 98.85) (end 110.5 98.85) (width 0.2) (layer "F.Cu") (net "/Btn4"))
 (segment (start 113.6 97.534316) (end 112.284315 98.85) (width 0.2) (layer "F.Cu") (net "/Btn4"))
 (segment (start 119.334314 106.5) (end 123.318628 102.515686) (width 0.2) (layer "F.Cu") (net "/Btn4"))
 (segment (start 112.602942 91.8) (end 113.6 92.797059) (width 0.2) (layer "F.Cu") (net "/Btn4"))
 (segment (start 118.700002 101) (end 117.700002 100) (width 0.2) (layer "F.Cu") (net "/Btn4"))
 (segment (start 91 92) (end 92.95 93.95) (width 0.2) (layer "F.Cu") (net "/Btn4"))
 (segment (start 115.905686 106.5) (end 119.334314 106.5) (width 0.2) (layer "F.Cu") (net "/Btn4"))
 (segment (start 110.5 98.85) (end 110.5 101.634316) (width 0.2) (layer "F.Cu") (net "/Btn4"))
 (segment (start 110.965684 102.1) (end 111.505686 102.1) (width 0.2) (layer "F.Cu") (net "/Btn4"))
 (segment (start 102.85 93.95) (end 105.000001 91.8) (width 0.2) (layer "F.Cu") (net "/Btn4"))
 (segment (start 123.318628 102.515686) (end 121.802942 101) (width 0.2) (layer "F.Cu") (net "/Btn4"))
 (segment (start 121.802942 101) (end 118.700002 101) (width 0.2) (layer "F.Cu") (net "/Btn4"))
 (segment (start 113.6 92.797059) (end 113.6 97.534316) (width 0.2) (layer "F.Cu") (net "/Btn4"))
 (segment (start 110.5 101.634316) (end 110.965684 102.1) (width 0.2) (layer "F.Cu") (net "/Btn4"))
 (segment (start 92.95 93.95) (end 102.85 93.95) (width 0.2) (layer "F.Cu") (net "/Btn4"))
 (segment (start 112.768628 91.4) (end 114 92.631372) (width 0.2) (layer "F.Cu") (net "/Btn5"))
 (segment (start 104.625686 91.4) (end 112.768628 91.4) (width 0.2) (layer "F.Cu") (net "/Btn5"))
 (segment (start 102.475686 93.55) (end 104.625686 91.4) (width 0.2) (layer "F.Cu") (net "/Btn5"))
 (segment (start 95.09 93.55) (end 102.475686 93.55) (width 0.2) (layer "F.Cu") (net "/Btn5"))
 (segment (start 93.54 92) (end 95.09 93.55) (width 0.2) (layer "F.Cu") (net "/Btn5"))
 (segment (start 114 92.631372) (end 114 97.700002) (width 0.2) (layer "F.Cu") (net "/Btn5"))
 (segment (start 114 97.700002) (end 111.700002 100) (width 0.2) (layer "F.Cu") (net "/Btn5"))
 (segment (start 112.934314 91) (end 125.5 103.565686) (width 0.2) (layer "F.Cu") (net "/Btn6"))
 (segment (start 135 103.4) (end 135 100) (width 0.2) (layer "F.Cu") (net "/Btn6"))
 (segment (start 96.08 92) (end 97.23 93.15) (width 0.2) (layer "F.Cu") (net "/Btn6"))
 (segment (start 97.23 93.15) (end 102.31 93.15) (width 0.2) (layer "F.Cu") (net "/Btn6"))
 (segment (start 129 109.4) (end 135 103.4) (width 0.2) (layer "F.Cu") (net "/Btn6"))
 (segment (start 104.46 91) (end 112.934314 91) (width 0.2) (layer "F.Cu") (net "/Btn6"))
 (segment (start 125.5 103.565686) (end 125.5 108.5) (width 0.2) (layer "F.Cu") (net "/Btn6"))
 (segment (start 125.5 108.5) (end 126.4 109.4) (width 0.2) (layer "F.Cu") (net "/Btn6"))
 (segment (start 126.4 109.4) (end 129 109.4) (width 0.2) (layer "F.Cu") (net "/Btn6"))
 (segment (start 102.31 93.15) (end 104.46 91) (width 0.2) (layer "F.Cu") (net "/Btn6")))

